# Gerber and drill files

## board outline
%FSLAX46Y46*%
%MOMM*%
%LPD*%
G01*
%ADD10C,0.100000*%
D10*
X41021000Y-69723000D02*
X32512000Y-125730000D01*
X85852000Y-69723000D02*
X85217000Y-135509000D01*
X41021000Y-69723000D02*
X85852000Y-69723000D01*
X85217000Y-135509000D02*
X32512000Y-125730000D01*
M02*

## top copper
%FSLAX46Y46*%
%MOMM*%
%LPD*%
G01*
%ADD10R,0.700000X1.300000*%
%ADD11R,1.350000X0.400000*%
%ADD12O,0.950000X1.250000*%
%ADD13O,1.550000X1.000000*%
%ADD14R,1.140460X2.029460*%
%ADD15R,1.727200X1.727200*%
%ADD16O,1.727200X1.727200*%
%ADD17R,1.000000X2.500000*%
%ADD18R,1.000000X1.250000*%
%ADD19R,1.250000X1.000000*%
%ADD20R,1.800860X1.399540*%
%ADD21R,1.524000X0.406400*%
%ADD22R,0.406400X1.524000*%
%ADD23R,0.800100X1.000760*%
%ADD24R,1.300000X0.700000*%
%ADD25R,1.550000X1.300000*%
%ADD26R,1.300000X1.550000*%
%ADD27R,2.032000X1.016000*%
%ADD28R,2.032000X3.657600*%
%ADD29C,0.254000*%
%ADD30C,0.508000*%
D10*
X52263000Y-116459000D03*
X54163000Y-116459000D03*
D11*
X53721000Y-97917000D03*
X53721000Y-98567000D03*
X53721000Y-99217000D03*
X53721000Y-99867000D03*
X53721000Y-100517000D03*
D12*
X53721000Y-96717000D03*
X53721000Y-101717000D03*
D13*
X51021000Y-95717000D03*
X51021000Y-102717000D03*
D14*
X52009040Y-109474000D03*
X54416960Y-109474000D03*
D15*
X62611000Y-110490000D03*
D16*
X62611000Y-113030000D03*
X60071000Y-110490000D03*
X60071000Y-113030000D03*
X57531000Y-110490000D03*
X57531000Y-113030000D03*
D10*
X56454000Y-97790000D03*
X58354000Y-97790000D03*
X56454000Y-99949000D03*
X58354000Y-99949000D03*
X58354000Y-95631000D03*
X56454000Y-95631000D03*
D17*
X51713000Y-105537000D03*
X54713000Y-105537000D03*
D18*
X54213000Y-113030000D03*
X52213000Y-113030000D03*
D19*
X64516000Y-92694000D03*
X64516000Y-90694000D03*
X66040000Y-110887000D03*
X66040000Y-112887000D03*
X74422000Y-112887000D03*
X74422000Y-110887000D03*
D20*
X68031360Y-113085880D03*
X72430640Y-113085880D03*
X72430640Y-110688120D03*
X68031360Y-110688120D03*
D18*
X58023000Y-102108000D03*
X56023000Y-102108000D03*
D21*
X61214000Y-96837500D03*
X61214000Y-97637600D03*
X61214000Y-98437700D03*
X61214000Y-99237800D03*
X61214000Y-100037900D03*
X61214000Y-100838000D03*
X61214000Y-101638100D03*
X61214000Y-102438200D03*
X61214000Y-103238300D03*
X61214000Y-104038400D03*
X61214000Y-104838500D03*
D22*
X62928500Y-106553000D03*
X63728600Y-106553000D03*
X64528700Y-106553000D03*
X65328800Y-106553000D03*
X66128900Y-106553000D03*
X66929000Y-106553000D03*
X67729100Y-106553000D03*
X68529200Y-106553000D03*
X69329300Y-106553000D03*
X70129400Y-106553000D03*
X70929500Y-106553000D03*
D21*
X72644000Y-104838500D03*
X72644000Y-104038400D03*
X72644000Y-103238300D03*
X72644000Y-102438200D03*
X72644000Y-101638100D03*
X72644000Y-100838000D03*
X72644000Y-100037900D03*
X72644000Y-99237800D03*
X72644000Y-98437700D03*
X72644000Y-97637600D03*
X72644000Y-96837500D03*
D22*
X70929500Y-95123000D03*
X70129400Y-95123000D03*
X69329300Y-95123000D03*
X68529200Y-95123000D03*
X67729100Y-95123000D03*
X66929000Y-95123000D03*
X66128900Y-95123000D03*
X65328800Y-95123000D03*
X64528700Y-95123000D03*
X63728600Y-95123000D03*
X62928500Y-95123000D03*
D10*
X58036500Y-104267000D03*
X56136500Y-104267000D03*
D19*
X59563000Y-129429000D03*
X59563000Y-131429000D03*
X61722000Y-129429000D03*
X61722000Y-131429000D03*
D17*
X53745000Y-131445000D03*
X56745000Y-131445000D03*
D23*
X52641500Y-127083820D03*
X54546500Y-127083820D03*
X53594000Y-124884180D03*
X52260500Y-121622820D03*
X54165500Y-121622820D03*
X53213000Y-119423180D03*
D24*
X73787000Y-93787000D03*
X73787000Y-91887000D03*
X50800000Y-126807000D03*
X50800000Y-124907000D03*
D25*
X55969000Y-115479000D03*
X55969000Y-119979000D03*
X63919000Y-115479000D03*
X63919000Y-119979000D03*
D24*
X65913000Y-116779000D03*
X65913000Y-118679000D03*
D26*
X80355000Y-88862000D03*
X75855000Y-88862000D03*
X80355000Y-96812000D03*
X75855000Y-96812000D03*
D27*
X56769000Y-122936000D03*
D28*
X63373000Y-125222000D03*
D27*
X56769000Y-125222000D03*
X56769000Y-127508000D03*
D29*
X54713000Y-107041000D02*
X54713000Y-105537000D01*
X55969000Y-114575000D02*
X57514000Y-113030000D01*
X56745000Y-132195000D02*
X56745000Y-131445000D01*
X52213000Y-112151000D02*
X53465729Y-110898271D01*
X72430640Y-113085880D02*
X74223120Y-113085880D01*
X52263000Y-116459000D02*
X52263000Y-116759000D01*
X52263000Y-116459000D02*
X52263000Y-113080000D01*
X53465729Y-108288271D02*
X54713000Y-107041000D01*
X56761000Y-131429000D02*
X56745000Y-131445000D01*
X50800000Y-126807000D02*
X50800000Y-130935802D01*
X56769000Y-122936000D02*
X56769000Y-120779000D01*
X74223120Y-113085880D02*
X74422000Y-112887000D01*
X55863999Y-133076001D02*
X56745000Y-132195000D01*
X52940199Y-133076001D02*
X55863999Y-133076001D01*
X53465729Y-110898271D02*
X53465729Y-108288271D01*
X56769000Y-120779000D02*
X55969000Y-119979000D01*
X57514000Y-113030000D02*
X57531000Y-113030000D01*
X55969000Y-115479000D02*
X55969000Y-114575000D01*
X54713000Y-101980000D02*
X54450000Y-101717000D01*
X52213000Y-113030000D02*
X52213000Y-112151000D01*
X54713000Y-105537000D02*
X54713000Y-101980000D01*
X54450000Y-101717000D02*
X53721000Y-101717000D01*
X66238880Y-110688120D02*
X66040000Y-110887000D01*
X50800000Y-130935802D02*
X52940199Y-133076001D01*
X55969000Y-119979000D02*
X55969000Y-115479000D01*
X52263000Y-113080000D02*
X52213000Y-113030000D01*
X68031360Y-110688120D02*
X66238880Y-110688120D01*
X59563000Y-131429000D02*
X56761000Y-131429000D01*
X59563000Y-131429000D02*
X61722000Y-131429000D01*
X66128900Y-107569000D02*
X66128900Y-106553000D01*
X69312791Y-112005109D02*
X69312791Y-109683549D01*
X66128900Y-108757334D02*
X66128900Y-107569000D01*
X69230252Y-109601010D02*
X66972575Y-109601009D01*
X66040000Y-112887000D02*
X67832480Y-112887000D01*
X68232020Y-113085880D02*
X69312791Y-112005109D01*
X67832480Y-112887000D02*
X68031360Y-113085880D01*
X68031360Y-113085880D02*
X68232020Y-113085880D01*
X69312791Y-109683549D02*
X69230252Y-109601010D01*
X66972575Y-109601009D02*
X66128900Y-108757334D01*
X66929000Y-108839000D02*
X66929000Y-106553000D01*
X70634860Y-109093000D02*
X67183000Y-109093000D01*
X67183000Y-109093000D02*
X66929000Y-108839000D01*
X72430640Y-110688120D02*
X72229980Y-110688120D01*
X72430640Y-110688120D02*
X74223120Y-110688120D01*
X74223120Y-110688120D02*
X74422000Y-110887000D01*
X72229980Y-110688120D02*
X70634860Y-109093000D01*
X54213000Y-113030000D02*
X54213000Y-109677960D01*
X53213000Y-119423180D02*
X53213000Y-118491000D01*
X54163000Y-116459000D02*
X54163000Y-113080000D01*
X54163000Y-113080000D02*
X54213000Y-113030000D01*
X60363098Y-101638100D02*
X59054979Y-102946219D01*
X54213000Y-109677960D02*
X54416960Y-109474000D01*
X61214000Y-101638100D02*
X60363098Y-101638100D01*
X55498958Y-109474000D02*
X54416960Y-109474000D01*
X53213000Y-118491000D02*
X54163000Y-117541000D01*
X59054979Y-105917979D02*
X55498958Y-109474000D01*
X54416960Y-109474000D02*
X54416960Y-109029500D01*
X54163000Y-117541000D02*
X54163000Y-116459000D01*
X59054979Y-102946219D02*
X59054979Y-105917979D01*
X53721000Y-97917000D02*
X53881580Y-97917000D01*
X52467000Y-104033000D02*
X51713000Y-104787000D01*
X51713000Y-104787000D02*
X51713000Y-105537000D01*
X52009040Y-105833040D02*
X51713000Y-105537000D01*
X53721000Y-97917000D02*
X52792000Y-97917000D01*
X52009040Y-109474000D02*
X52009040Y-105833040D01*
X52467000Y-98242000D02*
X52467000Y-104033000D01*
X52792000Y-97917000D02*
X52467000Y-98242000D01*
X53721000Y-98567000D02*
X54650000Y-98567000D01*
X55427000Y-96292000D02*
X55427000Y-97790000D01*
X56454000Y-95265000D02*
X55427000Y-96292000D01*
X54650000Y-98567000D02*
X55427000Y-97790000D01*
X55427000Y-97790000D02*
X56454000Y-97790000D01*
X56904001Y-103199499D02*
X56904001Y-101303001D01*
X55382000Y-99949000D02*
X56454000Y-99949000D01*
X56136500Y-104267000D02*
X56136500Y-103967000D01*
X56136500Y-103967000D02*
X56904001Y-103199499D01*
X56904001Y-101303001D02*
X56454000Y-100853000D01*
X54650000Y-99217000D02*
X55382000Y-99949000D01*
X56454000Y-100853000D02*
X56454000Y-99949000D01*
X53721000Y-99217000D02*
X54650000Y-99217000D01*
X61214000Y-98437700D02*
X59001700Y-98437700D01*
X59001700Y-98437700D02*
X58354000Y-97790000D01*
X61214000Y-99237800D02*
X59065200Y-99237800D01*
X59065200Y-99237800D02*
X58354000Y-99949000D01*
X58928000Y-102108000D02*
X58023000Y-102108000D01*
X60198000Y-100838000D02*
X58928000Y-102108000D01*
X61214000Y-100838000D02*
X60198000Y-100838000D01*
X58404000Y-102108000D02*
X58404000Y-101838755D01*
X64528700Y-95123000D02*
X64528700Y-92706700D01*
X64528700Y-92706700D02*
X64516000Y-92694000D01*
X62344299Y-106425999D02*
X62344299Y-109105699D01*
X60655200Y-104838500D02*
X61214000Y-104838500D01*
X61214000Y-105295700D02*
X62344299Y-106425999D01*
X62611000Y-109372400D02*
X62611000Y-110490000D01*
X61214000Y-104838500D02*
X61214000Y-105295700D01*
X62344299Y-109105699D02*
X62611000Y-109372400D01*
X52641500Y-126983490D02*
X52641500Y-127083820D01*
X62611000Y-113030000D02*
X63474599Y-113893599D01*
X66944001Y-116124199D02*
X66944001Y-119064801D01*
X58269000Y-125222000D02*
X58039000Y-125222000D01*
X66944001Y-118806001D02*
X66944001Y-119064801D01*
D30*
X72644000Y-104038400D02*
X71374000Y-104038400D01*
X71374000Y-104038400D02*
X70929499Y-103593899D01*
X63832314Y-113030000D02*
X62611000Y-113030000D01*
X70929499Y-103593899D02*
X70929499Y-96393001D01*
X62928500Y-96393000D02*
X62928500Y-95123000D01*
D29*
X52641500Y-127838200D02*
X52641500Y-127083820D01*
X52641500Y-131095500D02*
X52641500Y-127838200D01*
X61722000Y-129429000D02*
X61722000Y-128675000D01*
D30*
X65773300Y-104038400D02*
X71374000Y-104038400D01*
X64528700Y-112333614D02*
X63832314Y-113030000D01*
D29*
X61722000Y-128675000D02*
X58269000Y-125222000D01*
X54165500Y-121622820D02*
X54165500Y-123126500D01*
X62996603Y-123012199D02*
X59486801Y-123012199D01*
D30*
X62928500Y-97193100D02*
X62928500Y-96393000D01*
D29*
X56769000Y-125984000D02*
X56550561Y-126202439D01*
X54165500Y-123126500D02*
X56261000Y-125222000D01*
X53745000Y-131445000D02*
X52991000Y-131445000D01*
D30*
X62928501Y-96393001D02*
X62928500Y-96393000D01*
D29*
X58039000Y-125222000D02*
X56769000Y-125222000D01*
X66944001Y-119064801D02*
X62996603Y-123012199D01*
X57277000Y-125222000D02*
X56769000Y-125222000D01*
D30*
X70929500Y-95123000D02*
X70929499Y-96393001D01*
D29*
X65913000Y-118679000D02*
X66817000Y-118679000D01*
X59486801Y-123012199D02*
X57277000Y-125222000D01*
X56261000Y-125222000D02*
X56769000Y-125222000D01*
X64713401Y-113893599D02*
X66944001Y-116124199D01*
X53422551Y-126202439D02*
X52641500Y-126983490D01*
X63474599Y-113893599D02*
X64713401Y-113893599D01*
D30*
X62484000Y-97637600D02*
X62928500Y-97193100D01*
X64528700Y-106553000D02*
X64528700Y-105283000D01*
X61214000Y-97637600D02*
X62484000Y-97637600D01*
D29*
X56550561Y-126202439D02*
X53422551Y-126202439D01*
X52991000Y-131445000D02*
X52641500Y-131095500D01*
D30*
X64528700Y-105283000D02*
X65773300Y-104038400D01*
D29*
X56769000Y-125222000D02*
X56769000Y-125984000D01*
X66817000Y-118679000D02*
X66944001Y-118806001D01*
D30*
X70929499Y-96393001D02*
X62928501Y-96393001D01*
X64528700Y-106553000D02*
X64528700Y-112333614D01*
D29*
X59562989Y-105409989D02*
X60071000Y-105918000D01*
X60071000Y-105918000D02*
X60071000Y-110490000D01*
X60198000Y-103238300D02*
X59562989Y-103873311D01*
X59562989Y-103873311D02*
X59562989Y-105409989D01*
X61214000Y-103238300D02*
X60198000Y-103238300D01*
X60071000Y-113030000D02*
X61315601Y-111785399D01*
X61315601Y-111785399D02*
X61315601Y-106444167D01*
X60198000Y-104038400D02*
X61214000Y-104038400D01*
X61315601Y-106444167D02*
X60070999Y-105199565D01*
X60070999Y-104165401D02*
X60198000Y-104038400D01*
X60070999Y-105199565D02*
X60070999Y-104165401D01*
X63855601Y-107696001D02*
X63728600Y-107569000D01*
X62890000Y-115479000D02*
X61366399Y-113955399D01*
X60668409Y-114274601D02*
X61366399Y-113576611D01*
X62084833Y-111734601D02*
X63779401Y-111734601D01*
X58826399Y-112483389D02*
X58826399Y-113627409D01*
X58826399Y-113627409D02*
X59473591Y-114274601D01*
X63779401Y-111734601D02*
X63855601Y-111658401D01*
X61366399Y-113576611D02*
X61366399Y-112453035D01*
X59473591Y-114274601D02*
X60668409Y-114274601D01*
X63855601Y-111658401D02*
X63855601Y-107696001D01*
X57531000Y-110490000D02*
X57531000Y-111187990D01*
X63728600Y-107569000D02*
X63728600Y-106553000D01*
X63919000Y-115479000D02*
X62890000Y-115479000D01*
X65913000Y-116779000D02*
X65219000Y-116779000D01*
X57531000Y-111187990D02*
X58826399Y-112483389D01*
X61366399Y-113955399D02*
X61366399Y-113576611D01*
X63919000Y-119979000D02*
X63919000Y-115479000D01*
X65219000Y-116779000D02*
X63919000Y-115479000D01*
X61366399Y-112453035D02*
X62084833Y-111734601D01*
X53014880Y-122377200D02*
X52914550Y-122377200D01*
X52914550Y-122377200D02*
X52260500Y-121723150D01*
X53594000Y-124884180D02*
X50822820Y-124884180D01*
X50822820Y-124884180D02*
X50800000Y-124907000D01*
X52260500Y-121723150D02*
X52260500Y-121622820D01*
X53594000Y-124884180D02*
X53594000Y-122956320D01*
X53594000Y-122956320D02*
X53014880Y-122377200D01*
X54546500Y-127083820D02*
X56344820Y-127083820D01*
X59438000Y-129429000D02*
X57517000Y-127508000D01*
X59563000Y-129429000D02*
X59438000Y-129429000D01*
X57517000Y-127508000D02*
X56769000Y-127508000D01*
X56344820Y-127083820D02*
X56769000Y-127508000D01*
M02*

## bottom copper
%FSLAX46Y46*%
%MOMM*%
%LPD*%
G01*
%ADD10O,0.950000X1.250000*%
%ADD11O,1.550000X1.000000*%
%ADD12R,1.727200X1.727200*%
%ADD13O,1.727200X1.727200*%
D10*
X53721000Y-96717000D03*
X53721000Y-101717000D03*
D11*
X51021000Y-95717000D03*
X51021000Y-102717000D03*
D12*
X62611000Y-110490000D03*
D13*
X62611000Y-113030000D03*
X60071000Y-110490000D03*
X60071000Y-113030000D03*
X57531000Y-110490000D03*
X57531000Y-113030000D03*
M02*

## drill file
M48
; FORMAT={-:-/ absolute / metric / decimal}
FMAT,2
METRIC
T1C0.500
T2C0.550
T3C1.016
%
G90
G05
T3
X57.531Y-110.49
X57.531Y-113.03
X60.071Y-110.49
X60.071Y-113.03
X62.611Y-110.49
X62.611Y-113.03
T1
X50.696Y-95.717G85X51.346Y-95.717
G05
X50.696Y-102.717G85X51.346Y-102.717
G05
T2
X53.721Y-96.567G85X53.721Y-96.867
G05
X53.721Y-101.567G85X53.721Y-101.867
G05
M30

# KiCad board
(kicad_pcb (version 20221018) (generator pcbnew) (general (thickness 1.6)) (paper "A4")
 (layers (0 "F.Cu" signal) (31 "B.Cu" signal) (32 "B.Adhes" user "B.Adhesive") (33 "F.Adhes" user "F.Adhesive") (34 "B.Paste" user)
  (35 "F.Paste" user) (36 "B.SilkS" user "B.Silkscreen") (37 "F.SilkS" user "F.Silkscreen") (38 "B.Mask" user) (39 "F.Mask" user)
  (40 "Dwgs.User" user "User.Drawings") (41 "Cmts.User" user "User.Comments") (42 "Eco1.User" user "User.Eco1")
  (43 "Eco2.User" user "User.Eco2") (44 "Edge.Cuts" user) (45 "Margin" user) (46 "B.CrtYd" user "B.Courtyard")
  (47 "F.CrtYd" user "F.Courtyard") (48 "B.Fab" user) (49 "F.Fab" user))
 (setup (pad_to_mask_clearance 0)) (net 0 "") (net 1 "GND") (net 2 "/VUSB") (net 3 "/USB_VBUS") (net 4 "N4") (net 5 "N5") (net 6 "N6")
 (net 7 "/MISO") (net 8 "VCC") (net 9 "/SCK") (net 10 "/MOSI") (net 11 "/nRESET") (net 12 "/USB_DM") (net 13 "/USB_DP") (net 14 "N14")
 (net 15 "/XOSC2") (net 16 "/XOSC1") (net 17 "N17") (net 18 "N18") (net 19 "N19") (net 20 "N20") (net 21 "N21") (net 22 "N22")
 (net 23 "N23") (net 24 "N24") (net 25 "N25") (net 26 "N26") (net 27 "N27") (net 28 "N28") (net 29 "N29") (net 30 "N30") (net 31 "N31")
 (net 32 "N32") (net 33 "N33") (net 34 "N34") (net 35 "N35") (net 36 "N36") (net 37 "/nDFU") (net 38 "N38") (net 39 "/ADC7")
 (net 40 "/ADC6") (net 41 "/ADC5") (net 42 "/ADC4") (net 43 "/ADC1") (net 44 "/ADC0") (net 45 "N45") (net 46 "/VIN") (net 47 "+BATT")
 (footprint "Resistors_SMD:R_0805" (layer "F.Cu") (at 53.213 116.459)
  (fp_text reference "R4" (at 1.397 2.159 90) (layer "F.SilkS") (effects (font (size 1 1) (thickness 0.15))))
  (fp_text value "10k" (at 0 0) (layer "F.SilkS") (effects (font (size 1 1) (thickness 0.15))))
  (pad "1" smd rect (at -0.95 0) (size 0.7 1.3) (layers "F.Cu" "F.Paste" "F.Mask") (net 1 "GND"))
  (pad "2" smd rect (at 0.95 0) (size 0.7 1.3) (layers "F.Cu" "F.Paste" "F.Mask") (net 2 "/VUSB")))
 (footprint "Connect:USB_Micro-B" (layer "F.Cu") (at 53.721 97.917)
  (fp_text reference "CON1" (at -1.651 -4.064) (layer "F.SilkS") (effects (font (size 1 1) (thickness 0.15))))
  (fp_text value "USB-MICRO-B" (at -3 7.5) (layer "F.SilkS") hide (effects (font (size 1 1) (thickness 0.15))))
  (pad "1" smd rect (at 0 0) (size 1.35 0.4) (layers "F.Cu" "F.Paste" "F.Mask") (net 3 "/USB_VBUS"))
  (pad "2" smd rect (at 0 0.65) (size 1.35 0.4) (layers "F.Cu" "F.Paste" "F.Mask") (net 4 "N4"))
  (pad "3" smd rect (at 0 1.3) (size 1.35 0.4) (layers "F.Cu" "F.Paste" "F.Mask") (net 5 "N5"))
  (pad "4" smd rect (at 0 1.95) (size 1.35 0.4) (layers "F.Cu" "F.Paste" "F.Mask") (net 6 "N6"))
  (pad "5" smd rect (at 0 2.6) (size 1.35 0.4) (layers "F.Cu" "F.Paste" "F.Mask") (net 1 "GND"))
  (pad "6" thru_hole oval (at 0 -1.2) (size 0.95 1.25) (drill oval 0.55 0.85) (layers "*.Cu" "*.Mask" "F.SilkS") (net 1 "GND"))
  (pad "7" thru_hole oval (at 0 3.8) (size 0.95 1.25) (drill oval 0.55 0.85) (layers "*.Cu" "*.Mask" "F.SilkS") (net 1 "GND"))
  (pad "8" thru_hole oval (at -2.7 -2.2) (size 1.55 1) (drill oval 1.15 0.5) (layers "*.Cu" "*.Mask" "F.SilkS") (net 1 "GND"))
  (pad "9" thru_hole oval (at -2.7 4.8) (size 1.55 1) (drill oval 1.15 0.5) (layers "*.Cu" "*.Mask" "F.SilkS") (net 1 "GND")))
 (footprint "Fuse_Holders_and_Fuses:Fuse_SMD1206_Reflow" (layer "F.Cu") (at 53.213 109.474)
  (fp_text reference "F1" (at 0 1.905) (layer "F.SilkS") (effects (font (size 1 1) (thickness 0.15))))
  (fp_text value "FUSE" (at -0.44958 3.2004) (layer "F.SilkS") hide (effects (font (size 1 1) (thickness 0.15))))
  (pad "1" smd rect (at -1.20396 0 90) (size 2.02946 1.14046) (layers "F.Cu" "F.Paste" "F.Mask") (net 3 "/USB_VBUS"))
  (pad "2" smd rect (at 1.20396 0 90) (size 2.02946 1.14046) (layers "F.Cu" "F.Paste" "F.Mask") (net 2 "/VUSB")))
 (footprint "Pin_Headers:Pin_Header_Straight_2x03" (layer "F.Cu") (at 60.071 111.76 180)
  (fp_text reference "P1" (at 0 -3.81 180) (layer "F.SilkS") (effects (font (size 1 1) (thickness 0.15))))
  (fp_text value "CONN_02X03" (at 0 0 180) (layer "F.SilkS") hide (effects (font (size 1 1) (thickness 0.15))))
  (pad "1" thru_hole rect (at -2.54 1.27 180) (size 1.7272 1.7272) (drill 1.016) (layers "*.Cu" "*.Mask" "F.SilkS") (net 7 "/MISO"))
  (pad "2" thru_hole oval (at -2.54 -1.27 180) (size 1.7272 1.7272) (drill 1.016) (layers "*.Cu" "*.Mask" "F.SilkS") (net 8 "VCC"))
  (pad "3" thru_hole oval (at 0 1.27 180) (size 1.7272 1.7272) (drill 1.016) (layers "*.Cu" "*.Mask" "F.SilkS") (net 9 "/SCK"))
  (pad "4" thru_hole oval (at 0 -1.27 180) (size 1.7272 1.7272) (drill 1.016) (layers "*.Cu" "*.Mask" "F.SilkS") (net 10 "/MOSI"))
  (pad "5" thru_hole oval (at 2.54 1.27 180) (size 1.7272 1.7272) (drill 1.016) (layers "*.Cu" "*.Mask" "F.SilkS") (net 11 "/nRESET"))
  (pad "6" thru_hole oval (at 2.54 -1.27 180) (size 1.7272 1.7272) (drill 1.016) (layers "*.Cu" "*.Mask" "F.SilkS") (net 1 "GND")))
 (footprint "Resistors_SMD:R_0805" (layer "F.Cu") (at 57.404 97.79)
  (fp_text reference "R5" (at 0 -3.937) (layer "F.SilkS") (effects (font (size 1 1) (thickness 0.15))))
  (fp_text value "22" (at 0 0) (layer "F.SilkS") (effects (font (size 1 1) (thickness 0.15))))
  (pad "1" smd rect (at -0.95 0) (size 0.7 1.3) (layers "F.Cu" "F.Paste" "F.Mask") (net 4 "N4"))
  (pad "2" smd rect (at 0.95 0) (size 0.7 1.3) (layers "F.Cu" "F.Paste" "F.Mask") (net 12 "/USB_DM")))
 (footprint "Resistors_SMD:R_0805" (layer "F.Cu") (at 57.404 99.949)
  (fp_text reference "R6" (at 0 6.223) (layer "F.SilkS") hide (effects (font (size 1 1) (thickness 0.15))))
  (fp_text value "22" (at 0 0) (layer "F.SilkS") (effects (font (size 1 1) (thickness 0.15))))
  (pad "1" smd rect (at -0.95 0) (size 0.7 1.3) (layers "F.Cu" "F.Paste" "F.Mask") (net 5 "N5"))
  (pad "2" smd rect (at 0.95 0) (size 0.7 1.3) (layers "F.Cu" "F.Paste" "F.Mask") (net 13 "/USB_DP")))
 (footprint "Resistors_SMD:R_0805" (layer "F.Cu") (at 57.404 95.631 180)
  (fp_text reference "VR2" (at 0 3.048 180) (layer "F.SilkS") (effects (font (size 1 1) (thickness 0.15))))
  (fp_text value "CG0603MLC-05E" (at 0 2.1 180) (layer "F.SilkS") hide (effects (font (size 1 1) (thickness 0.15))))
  (pad "1" smd rect (at -0.95 0 180) (size 0.7 1.3) (layers "F.Cu" "F.Paste" "F.Mask") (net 1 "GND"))
  (pad "2" smd rect (at 0.95 0 180) (size 0.7 1.3) (layers "F.Cu" "F.Paste" "F.Mask") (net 4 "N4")))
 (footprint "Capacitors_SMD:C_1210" (layer "F.Cu") (at 53.213 105.537)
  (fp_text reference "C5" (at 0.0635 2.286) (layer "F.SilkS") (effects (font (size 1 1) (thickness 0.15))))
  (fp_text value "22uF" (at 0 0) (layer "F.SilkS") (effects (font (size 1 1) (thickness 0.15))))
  (pad "1" smd rect (at -1.5 0) (size 1 2.5) (layers "F.Cu" "F.Paste" "F.Mask") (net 3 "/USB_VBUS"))
  (pad "2" smd rect (at 1.5 0) (size 1 2.5) (layers "F.Cu" "F.Paste" "F.Mask") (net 1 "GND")))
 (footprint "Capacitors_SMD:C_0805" (layer "F.Cu") (at 53.213 113.03 180)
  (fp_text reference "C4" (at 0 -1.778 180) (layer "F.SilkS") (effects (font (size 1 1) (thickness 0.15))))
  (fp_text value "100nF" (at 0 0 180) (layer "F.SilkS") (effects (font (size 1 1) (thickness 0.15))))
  (pad "1" smd rect (at -1 0 180) (size 1 1.25) (layers "F.Cu" "F.Paste" "F.Mask") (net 2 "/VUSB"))
  (pad "2" smd rect (at 1 0 180) (size 1 1.25) (layers "F.Cu" "F.Paste" "F.Mask") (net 1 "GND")))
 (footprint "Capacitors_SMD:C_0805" (layer "F.Cu") (at 64.516 91.694 90)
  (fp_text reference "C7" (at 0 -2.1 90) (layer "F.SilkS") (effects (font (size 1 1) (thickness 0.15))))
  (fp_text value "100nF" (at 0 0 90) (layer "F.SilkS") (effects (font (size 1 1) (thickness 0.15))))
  (pad "1" smd rect (at -1 0 90) (size 1 1.25) (layers "F.Cu" "F.Paste" "F.Mask") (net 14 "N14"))
  (pad "2" smd rect (at 1 0 90) (size 1 1.25) (layers "F.Cu" "F.Paste" "F.Mask") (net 1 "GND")))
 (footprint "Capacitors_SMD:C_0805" (layer "F.Cu") (at 66.04 111.887 -90)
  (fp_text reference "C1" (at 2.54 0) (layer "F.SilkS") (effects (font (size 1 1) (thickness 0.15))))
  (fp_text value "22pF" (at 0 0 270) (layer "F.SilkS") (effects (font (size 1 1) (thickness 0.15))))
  (pad "1" smd rect (at -1 0 270) (size 1 1.25) (layers "F.Cu" "F.Paste" "F.Mask") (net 1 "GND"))
  (pad "2" smd rect (at 1 0 270) (size 1 1.25) (layers "F.Cu" "F.Paste" "F.Mask") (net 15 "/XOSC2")))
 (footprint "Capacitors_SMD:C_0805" (layer "F.Cu") (at 74.422 111.887 90)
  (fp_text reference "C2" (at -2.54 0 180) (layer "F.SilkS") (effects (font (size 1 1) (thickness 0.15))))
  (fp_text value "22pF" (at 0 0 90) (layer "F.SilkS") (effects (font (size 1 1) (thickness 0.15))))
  (pad "1" smd rect (at -1 0 90) (size 1 1.25) (layers "F.Cu" "F.Paste" "F.Mask") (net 1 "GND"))
  (pad "2" smd rect (at 1 0 90) (size 1 1.25) (layers "F.Cu" "F.Paste" "F.Mask") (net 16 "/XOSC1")))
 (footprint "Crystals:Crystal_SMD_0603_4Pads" (layer "F.Cu") (at 70.231 111.887)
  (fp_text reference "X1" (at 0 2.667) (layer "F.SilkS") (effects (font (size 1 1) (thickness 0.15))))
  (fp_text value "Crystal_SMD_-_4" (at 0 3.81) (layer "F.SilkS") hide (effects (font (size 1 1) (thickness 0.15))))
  (pad "1" smd rect (at -2.19964 1.19888) (size 1.80086 1.39954) (layers "F.Cu" "F.Paste" "F.Mask") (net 15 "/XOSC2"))
  (pad "2" smd rect (at 2.19964 1.19888) (size 1.80086 1.39954) (layers "F.Cu" "F.Paste" "F.Mask") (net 1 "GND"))
  (pad "3" smd rect (at 2.19964 -1.19888) (size 1.80086 1.39954) (layers "F.Cu" "F.Paste" "F.Mask") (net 16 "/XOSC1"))
  (pad "4" smd rect (at -2.19964 -1.19888) (size 1.80086 1.39954) (layers "F.Cu" "F.Paste" "F.Mask") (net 1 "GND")))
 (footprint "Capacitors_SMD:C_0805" (layer "F.Cu") (at 57.023 102.108 180)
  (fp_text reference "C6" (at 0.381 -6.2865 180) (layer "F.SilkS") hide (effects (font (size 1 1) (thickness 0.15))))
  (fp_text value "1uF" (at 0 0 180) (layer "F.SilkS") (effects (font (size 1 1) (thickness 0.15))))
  (pad "1" smd rect (at -1 0 180) (size 1 1.25) (layers "F.Cu" "F.Paste" "F.Mask") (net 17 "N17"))
  (pad "2" smd rect (at 1 0 180) (size 1 1.25) (layers "F.Cu" "F.Paste" "F.Mask") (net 1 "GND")))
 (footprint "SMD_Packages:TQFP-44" (layer "F.Cu") (at 66.929 100.838)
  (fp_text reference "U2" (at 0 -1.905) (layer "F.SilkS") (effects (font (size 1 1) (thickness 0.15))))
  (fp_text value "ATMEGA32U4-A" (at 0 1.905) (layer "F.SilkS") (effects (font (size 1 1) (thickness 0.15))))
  (pad "1" smd rect (at -5.715 -4.0005) (size 1.524 0.4064) (layers "F.Cu" "F.Paste" "F.Mask") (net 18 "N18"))
  (pad "2" smd rect (at -5.715 -3.2004) (size 1.524 0.4064) (layers "F.Cu" "F.Paste" "F.Mask") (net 8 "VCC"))
  (pad "3" smd rect (at -5.715 -2.4003) (size 1.524 0.4064) (layers "F.Cu" "F.Paste" "F.Mask") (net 12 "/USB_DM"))
  (pad "4" smd rect (at -5.715 -1.6002) (size 1.524 0.4064) (layers "F.Cu" "F.Paste" "F.Mask") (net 13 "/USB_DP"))
  (pad "5" smd rect (at -5.715 -0.8001) (size 1.524 0.4064) (layers "F.Cu" "F.Paste" "F.Mask") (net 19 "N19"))
  (pad "6" smd rect (at -5.715 0) (size 1.524 0.4064) (layers "F.Cu" "F.Paste" "F.Mask") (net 17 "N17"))
  (pad "7" smd rect (at -5.715 0.8001) (size 1.524 0.4064) (layers "F.Cu" "F.Paste" "F.Mask") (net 2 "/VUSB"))
  (pad "8" smd rect (at -5.715 1.6002) (size 1.524 0.4064) (layers "F.Cu" "F.Paste" "F.Mask") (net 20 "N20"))
  (pad "9" smd rect (at -5.715 2.4003) (size 1.524 0.4064) (layers "F.Cu" "F.Paste" "F.Mask") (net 9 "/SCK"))
  (pad "10" smd rect (at -5.715 3.2004) (size 1.524 0.4064) (layers "F.Cu" "F.Paste" "F.Mask") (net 10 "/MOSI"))
  (pad "11" smd rect (at -5.715 4.0005) (size 1.524 0.4064) (layers "F.Cu" "F.Paste" "F.Mask") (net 7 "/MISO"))
  (pad "12" smd rect (at -4.0005 5.715) (size 0.4064 1.524) (layers "F.Cu" "F.Paste" "F.Mask") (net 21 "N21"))
  (pad "13" smd rect (at -3.2004 5.715) (size 0.4064 1.524) (layers "F.Cu" "F.Paste" "F.Mask") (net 11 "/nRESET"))
  (pad "14" smd rect (at -2.4003 5.715) (size 0.4064 1.524) (layers "F.Cu" "F.Paste" "F.Mask") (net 8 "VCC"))
  (pad "15" smd rect (at -1.6002 5.715) (size 0.4064 1.524) (layers "F.Cu" "F.Paste" "F.Mask") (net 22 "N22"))
  (pad "16" smd rect (at -0.8001 5.715) (size 0.4064 1.524) (layers "F.Cu" "F.Paste" "F.Mask") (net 15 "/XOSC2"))
  (pad "17" smd rect (at 0 5.715) (size 0.4064 1.524) (layers "F.Cu" "F.Paste" "F.Mask") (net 16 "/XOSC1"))
  (pad "18" smd rect (at 0.8001 5.715) (size 0.4064 1.524) (layers "F.Cu" "F.Paste" "F.Mask") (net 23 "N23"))
  (pad "19" smd rect (at 1.6002 5.715) (size 0.4064 1.524) (layers "F.Cu" "F.Paste" "F.Mask") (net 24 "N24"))
  (pad "20" smd rect (at 2.4003 5.715) (size 0.4064 1.524) (layers "F.Cu" "F.Paste" "F.Mask") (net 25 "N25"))
  (pad "21" smd rect (at 3.2004 5.715) (size 0.4064 1.524) (layers "F.Cu" "F.Paste" "F.Mask") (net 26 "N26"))
  (pad "22" smd rect (at 4.0005 5.715) (size 0.4064 1.524) (layers "F.Cu" "F.Paste" "F.Mask") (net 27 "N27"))
  (pad "23" smd rect (at 5.715 4.0005) (size 1.524 0.4064) (layers "F.Cu" "F.Paste" "F.Mask") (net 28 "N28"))
  (pad "24" smd rect (at 5.715 3.2004) (size 1.524 0.4064) (layers "F.Cu" "F.Paste" "F.Mask") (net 8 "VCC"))
  (pad "25" smd rect (at 5.715 2.4003) (size 1.524 0.4064) (layers "F.Cu" "F.Paste" "F.Mask") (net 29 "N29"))
  (pad "26" smd rect (at 5.715 1.6002) (size 1.524 0.4064) (layers "F.Cu" "F.Paste" "F.Mask") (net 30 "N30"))
  (pad "27" smd rect (at 5.715 0.8001) (size 1.524 0.4064) (layers "F.Cu" "F.Paste" "F.Mask") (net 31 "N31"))
  (pad "28" smd rect (at 5.715 0) (size 1.524 0.4064) (layers "F.Cu" "F.Paste" "F.Mask") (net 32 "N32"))
  (pad "29" smd rect (at 5.715 -0.8001) (size 1.524 0.4064) (layers "F.Cu" "F.Paste" "F.Mask") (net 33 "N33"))
  (pad "30" smd rect (at 5.715 -1.6002) (size 1.524 0.4064) (layers "F.Cu" "F.Paste" "F.Mask") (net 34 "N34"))
  (pad "31" smd rect (at 5.715 -2.4003) (size 1.524 0.4064) (layers "F.Cu" "F.Paste" "F.Mask") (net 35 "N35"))
  (pad "32" smd rect (at 5.715 -3.2004) (size 1.524 0.4064) (layers "F.Cu" "F.Paste" "F.Mask") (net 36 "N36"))
  (pad "33" smd rect (at 5.715 -4.0005) (size 1.524 0.4064) (layers "F.Cu" "F.Paste" "F.Mask") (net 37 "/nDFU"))
  (pad "34" smd rect (at 4.0005 -5.715) (size 0.4064 1.524) (layers "F.Cu" "F.Paste" "F.Mask") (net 8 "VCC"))
  (pad "35" smd rect (at 3.2004 -5.715) (size 0.4064 1.524) (layers "F.Cu" "F.Paste" "F.Mask") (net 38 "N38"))
  (pad "36" smd rect (at 2.4003 -5.715) (size 0.4064 1.524) (layers "F.Cu" "F.Paste" "F.Mask") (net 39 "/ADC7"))
  (pad "37" smd rect (at 1.6002 -5.715) (size 0.4064 1.524) (layers "F.Cu" "F.Paste" "F.Mask") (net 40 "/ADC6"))
  (pad "38" smd rect (at 0.8001 -5.715) (size 0.4064 1.524) (layers "F.Cu" "F.Paste" "F.Mask") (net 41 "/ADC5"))
  (pad "39" smd rect (at 0 -5.715) (size 0.4064 1.524) (layers "F.Cu" "F.Paste" "F.Mask") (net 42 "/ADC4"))
  (pad "40" smd rect (at -0.8001 -5.715) (size 0.4064 1.524) (layers "F.Cu" "F.Paste" "F.Mask") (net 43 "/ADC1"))
  (pad "41" smd rect (at -1.6002 -5.715) (size 0.4064 1.524) (layers "F.Cu" "F.Paste" "F.Mask") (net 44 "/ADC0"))
  (pad "42" smd rect (at -2.4003 -5.715) (size 0.4064 1.524) (layers "F.Cu" "F.Paste" "F.Mask") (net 14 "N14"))
  (pad "43" smd rect (at -3.2004 -5.715) (size 0.4064 1.524) (layers "F.Cu" "F.Paste" "F.Mask") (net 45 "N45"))
  (pad "44" smd rect (at -4.0005 -5.715) (size 0.4064 1.524) (layers "F.Cu" "F.Paste" "F.Mask") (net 8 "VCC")))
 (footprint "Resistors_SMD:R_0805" (layer "F.Cu") (at 57.0865 104.267 180)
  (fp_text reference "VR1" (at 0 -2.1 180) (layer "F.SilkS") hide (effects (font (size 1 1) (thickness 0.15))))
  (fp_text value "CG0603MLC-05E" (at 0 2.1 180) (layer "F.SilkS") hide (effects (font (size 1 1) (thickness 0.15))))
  (pad "1" smd rect (at -0.95 0 180) (size 0.7 1.3) (layers "F.Cu" "F.Paste" "F.Mask") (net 1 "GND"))
  (pad "2" smd rect (at 0.95 0 180) (size 0.7 1.3) (layers "F.Cu" "F.Paste" "F.Mask") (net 5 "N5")))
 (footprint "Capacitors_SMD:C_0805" (layer "F.Cu") (at 59.563 130.429 -90)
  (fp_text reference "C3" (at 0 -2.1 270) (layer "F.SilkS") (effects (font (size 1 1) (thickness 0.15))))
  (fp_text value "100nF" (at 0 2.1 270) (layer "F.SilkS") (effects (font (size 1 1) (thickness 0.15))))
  (pad "1" smd rect (at -1 0 270) (size 1 1.25) (layers "F.Cu" "F.Paste" "F.Mask") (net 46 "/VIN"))
  (pad "2" smd rect (at 1 0 270) (size 1 1.25) (layers "F.Cu" "F.Paste" "F.Mask") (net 1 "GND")))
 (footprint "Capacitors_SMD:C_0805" (layer "F.Cu") (at 61.722 130.429 -90)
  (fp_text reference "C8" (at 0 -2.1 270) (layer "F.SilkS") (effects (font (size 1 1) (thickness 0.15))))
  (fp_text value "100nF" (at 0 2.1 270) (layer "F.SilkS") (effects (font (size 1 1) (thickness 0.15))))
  (pad "1" smd rect (at -1 0 270) (size 1 1.25) (layers "F.Cu" "F.Paste" "F.Mask") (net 8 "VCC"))
  (pad "2" smd rect (at 1 0 270) (size 1 1.25) (layers "F.Cu" "F.Paste" "F.Mask") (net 1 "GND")))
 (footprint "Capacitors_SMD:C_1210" (layer "F.Cu") (at 55.245 131.445)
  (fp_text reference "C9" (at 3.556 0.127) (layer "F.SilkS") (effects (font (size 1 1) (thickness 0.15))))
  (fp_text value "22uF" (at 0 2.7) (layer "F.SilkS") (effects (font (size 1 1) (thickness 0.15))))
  (pad "1" smd rect (at -1.5 0) (size 1 2.5) (layers "F.Cu" "F.Paste" "F.Mask") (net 8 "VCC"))
  (pad "2" smd rect (at 1.5 0) (size 1 2.5) (layers "F.Cu" "F.Paste" "F.Mask") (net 1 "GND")))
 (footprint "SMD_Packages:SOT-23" (layer "F.Cu") (at 53.594 125.984)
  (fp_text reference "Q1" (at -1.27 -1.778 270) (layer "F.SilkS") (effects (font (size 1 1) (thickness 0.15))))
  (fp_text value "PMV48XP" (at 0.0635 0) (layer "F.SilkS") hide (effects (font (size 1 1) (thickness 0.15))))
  (pad "1" smd rect (at -0.9525 1.09982) (size 0.8001 1.00076) (layers "F.Cu" "F.Paste" "F.Mask") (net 8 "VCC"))
  (pad "2" smd rect (at 0.9525 1.09982) (size 0.8001 1.00076) (layers "F.Cu" "F.Paste" "F.Mask") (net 46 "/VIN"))
  (pad "3" smd rect (at 0 -1.09982) (size 0.8001 1.00076) (layers "F.Cu" "F.Paste" "F.Mask") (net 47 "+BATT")))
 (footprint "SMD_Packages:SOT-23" (layer "F.Cu") (at 53.213 120.523)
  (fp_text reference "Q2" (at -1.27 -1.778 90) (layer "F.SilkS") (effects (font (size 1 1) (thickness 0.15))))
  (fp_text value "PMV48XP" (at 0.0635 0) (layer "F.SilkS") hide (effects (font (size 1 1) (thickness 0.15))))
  (pad "1" smd rect (at -0.9525 1.09982) (size 0.8001 1.00076) (layers "F.Cu" "F.Paste" "F.Mask") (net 47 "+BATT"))
  (pad "2" smd rect (at 0.9525 1.09982) (size 0.8001 1.00076) (layers "F.Cu" "F.Paste" "F.Mask") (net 8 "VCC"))
  (pad "3" smd rect (at 0 -1.09982) (size 0.8001 1.00076) (layers "F.Cu" "F.Paste" "F.Mask") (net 2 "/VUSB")))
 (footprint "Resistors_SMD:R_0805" (layer "F.Cu") (at 73.787 92.837 90)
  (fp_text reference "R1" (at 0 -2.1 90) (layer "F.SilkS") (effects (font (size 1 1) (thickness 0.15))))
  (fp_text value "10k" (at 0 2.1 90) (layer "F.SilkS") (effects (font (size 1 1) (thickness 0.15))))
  (pad "1" smd rect (at -0.95 0 90) (size 0.7 1.3) (layers "F.Cu" "F.Paste" "F.Mask") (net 37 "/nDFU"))
  (pad "2" smd rect (at 0.95 0 90) (size 0.7 1.3) (layers "F.Cu" "F.Paste" "F.Mask") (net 8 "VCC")))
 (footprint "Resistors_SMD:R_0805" (layer "F.Cu") (at 50.8 125.857 90)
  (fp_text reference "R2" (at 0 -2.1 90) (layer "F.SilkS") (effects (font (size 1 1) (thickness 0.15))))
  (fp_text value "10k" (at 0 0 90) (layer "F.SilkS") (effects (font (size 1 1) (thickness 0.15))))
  (pad "1" smd rect (at -0.95 0 90) (size 0.7 1.3) (layers "F.Cu" "F.Paste" "F.Mask") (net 1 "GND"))
  (pad "2" smd rect (at 0.95 0 90) (size 0.7 1.3) (layers "F.Cu" "F.Paste" "F.Mask") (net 47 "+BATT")))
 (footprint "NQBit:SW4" (layer "F.Cu") (at 59.944 117.729)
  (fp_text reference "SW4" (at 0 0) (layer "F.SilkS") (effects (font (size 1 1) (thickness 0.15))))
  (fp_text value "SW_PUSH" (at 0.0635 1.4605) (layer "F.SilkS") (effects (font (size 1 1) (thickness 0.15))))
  (pad "1" smd rect (at -3.975 -2.25) (size 1.55 1.3) (layers "F.Cu" "F.Paste" "F.Mask") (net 1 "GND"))
  (pad "1" smd rect (at -3.975 2.25) (size 1.55 1.3) (layers "F.Cu" "F.Paste" "F.Mask") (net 1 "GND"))
  (pad "2" smd rect (at 3.975 -2.25) (size 1.55 1.3) (layers "F.Cu" "F.Paste" "F.Mask") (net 11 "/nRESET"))
  (pad "2" smd rect (at 3.975 2.25) (size 1.55 1.3) (layers "F.Cu" "F.Paste" "F.Mask") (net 11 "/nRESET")))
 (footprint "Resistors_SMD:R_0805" (layer "F.Cu") (at 65.913 117.729 -90)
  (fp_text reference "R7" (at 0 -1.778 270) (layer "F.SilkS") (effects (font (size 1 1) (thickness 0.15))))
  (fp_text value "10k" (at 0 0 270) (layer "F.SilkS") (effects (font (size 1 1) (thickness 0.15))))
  (pad "1" smd rect (at -0.95 0 270) (size 0.7 1.3) (layers "F.Cu" "F.Paste" "F.Mask") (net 11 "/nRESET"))
  (pad "2" smd rect (at 0.95 0 270) (size 0.7 1.3) (layers "F.Cu" "F.Paste" "F.Mask") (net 8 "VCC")))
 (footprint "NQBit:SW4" (layer "F.Cu") (at 78.105 92.837 -90)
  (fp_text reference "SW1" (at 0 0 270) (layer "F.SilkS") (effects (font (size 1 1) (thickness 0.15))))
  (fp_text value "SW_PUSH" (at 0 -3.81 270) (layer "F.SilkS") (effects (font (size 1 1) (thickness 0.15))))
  (pad "1" smd rect (at -3.975 -2.25 270) (size 1.55 1.3) (layers "F.Cu" "F.Paste" "F.Mask") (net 1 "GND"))
  (pad "1" smd rect (at -3.975 2.25 270) (size 1.55 1.3) (layers "F.Cu" "F.Paste" "F.Mask") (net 1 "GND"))
  (pad "2" smd rect (at 3.975 -2.25 270) (size 1.55 1.3) (layers "F.Cu" "F.Paste" "F.Mask") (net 37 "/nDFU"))
  (pad "2" smd rect (at 3.975 2.25 270) (size 1.55 1.3) (layers "F.Cu" "F.Paste" "F.Mask") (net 37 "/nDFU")))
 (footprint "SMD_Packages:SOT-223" (layer "F.Cu") (at 60.071 125.222 -90)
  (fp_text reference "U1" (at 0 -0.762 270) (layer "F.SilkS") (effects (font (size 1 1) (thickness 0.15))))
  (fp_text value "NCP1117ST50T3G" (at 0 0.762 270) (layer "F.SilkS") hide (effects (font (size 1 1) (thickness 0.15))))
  (pad "1" smd rect (at -2.286 3.302 270) (size 1.016 2.032) (layers "F.Cu" "F.Paste" "F.Mask") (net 1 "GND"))
  (pad "2" smd rect (at 0 -3.302 270) (size 3.6576 2.032) (layers "F.Cu" "F.Paste" "F.Mask"))
  (pad "2" smd rect (at 0 3.302 270) (size 1.016 2.032) (layers "F.Cu" "F.Paste" "F.Mask") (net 8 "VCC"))
  (pad "3" smd rect (at 2.286 3.302 270) (size 1.016 2.032) (layers "F.Cu" "F.Paste" "F.Mask") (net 46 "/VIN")))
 (gr_line (start 41.021 69.723) (end 32.512 125.73) (stroke (width 0.1) (type solid)) (layer "Edge.Cuts"))
 (gr_line (start 85.852 69.723) (end 85.217 135.509) (stroke (width 0.1) (type solid)) (layer "Edge.Cuts"))
 (gr_line (start 41.021 69.723) (end 85.852 69.723) (stroke (width 0.1) (type solid)) (layer "Edge.Cuts"))
 (gr_line (start 85.217 135.509) (end 32.512 125.73) (stroke (width 0.1) (type solid)) (layer "Edge.Cuts"))
 (segment (start 54.713 107.041) (end 54.713 105.537) (width 0.254) (layer "F.Cu") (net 1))
 (segment (start 55.969 114.575) (end 57.514 113.03) (width 0.254) (layer "F.Cu") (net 1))
 (segment (start 56.745 132.195) (end 56.745 131.445) (width 0.254) (layer "F.Cu") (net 1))
 (segment (start 52.213 112.151) (end 53.465729 110.898271) (width 0.254) (layer "F.Cu") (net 1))
 (segment (start 72.43064 113.08588) (end 74.22312 113.08588) (width 0.254) (layer "F.Cu") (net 1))
 (segment (start 52.263 116.459) (end 52.263 116.759) (width 0.254) (layer "F.Cu") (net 1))
 (segment (start 52.263 116.459) (end 52.263 113.08) (width 0.254) (layer "F.Cu") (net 1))
 (segment (start 53.465729 108.288271) (end 54.713 107.041) (width 0.254) (layer "F.Cu") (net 1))
 (segment (start 56.761 131.429) (end 56.745 131.445) (width 0.254) (layer "F.Cu") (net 1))
 (segment (start 50.8 126.807) (end 50.8 130.935802) (width 0.254) (layer "F.Cu") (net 1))
 (segment (start 56.769 122.936) (end 56.769 120.779) (width 0.254) (layer "F.Cu") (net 1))
 (segment (start 74.22312 113.08588) (end 74.422 112.887) (width 0.254) (layer "F.Cu") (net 1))
 (segment (start 55.863999 133.076001) (end 56.745 132.195) (width 0.254) (layer "F.Cu") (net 1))
 (segment (start 52.940199 133.076001) (end 55.863999 133.076001) (width 0.254) (layer "F.Cu") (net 1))
 (segment (start 53.465729 110.898271) (end 53.465729 108.288271) (width 0.254) (layer "F.Cu") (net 1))
 (segment (start 56.769 120.779) (end 55.969 119.979) (width 0.254) (layer "F.Cu") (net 1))
 (segment (start 57.514 113.03) (end 57.531 113.03) (width 0.254) (layer "F.Cu") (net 1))
 (segment (start 55.969 115.479) (end 55.969 114.575) (width 0.254) (layer "F.Cu") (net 1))
 (segment (start 54.713 101.98) (end 54.45 101.717) (width 0.254) (layer "F.Cu") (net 1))
 (segment (start 52.213 113.03) (end 52.213 112.151) (width 0.254) (layer "F.Cu") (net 1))
 (segment (start 54.713 105.537) (end 54.713 101.98) (width 0.254) (layer "F.Cu") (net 1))
 (segment (start 54.45 101.717) (end 53.721 101.717) (width 0.254) (layer "F.Cu") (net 1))
 (segment (start 66.23888 110.68812) (end 66.04 110.887) (width 0.254) (layer "F.Cu") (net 1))
 (segment (start 50.8 130.935802) (end 52.940199 133.076001) (width 0.254) (layer "F.Cu") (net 1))
 (segment (start 55.969 119.979) (end 55.969 115.479) (width 0.254) (layer "F.Cu") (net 1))
 (segment (start 52.263 113.08) (end 52.213 113.03) (width 0.254) (layer "F.Cu") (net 1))
 (segment (start 68.03136 110.68812) (end 66.23888 110.68812) (width 0.254) (layer "F.Cu") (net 1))
 (segment (start 59.563 131.429) (end 56.761 131.429) (width 0.254) (layer "F.Cu") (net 1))
 (segment (start 59.563 131.429) (end 61.722 131.429) (width 0.254) (layer "F.Cu") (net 1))
 (segment (start 66.1289 107.569) (end 66.1289 106.553) (width 0.254) (layer "F.Cu") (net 15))
 (segment (start 69.312791 112.005109) (end 69.312791 109.683549) (width 0.254) (layer "F.Cu") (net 15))
 (segment (start 66.1289 108.757334) (end 66.1289 107.569) (width 0.254) (layer "F.Cu") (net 15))
 (segment (start 69.230252 109.60101) (end 66.972575 109.601009) (width 0.254) (layer "F.Cu") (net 15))
 (segment (start 66.04 112.887) (end 67.83248 112.887) (width 0.254) (layer "F.Cu") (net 15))
 (segment (start 68.23202 113.08588) (end 69.312791 112.005109) (width 0.254) (layer "F.Cu") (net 15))
 (segment (start 67.83248 112.887) (end 68.03136 113.08588) (width 0.254) (layer "F.Cu") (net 15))
 (segment (start 68.03136 113.08588) (end 68.23202 113.08588) (width 0.254) (layer "F.Cu") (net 15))
 (segment (start 69.312791 109.683549) (end 69.230252 109.60101) (width 0.254) (layer "F.Cu") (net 15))
 (segment (start 66.972575 109.601009) (end 66.1289 108.757334) (width 0.254) (layer "F.Cu") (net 15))
 (segment (start 66.929 108.839) (end 66.929 106.553) (width 0.254) (layer "F.Cu") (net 16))
 (segment (start 70.63486 109.093) (end 67.183 109.093) (width 0.254) (layer "F.Cu") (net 16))
 (segment (start 67.183 109.093) (end 66.929 108.839) (width 0.254) (layer "F.Cu") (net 16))
 (segment (start 72.43064 110.68812) (end 72.22998 110.68812) (width 0.254) (layer "F.Cu") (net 16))
 (segment (start 72.43064 110.68812) (end 74.22312 110.68812) (width 0.254) (layer "F.Cu") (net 16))
 (segment (start 74.22312 110.68812) (end 74.422 110.887) (width 0.254) (layer "F.Cu") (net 16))
 (segment (start 72.22998 110.68812) (end 70.63486 109.093) (width 0.254) (layer "F.Cu") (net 16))
 (segment (start 54.213 113.03) (end 54.213 109.67796) (width 0.254) (layer "F.Cu") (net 2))
 (segment (start 53.213 119.42318) (end 53.213 118.491) (width 0.254) (layer "F.Cu") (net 2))
 (segment (start 54.163 116.459) (end 54.163 113.08) (width 0.254) (layer "F.Cu") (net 2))
 (segment (start 54.163 113.08) (end 54.213 113.03) (width 0.254) (layer "F.Cu") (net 2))
 (segment (start 60.363098 101.6381) (end 59.054979 102.946219) (width 0.254) (layer "F.Cu") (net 2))
 (segment (start 54.213 109.67796) (end 54.41696 109.474) (width 0.254) (layer "F.Cu") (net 2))
 (segment (start 61.214 101.6381) (end 60.363098 101.6381) (width 0.254) (layer "F.Cu") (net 2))
 (segment (start 55.498958 109.474) (end 54.41696 109.474) (width 0.254) (layer "F.Cu") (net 2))
 (segment (start 53.213 118.491) (end 54.163 117.541) (width 0.254) (layer "F.Cu") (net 2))
 (segment (start 59.054979 105.917979) (end 55.498958 109.474) (width 0.254) (layer "F.Cu") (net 2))
 (segment (start 54.41696 109.474) (end 54.41696 109.0295) (width 0.254) (layer "F.Cu") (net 2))
 (segment (start 54.163 117.541) (end 54.163 116.459) (width 0.254) (layer "F.Cu") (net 2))
 (segment (start 59.054979 102.946219) (end 59.054979 105.917979) (width 0.254) (layer "F.Cu") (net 2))
 (segment (start 53.721 97.917) (end 53.88158 97.917) (width 0.254) (layer "F.Cu") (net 3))
 (segment (start 52.467 104.033) (end 51.713 104.787) (width 0.254) (layer "F.Cu") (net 3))
 (segment (start 51.713 104.787) (end 51.713 105.537) (width 0.254) (layer "F.Cu") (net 3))
 (segment (start 52.00904 105.83304) (end 51.713 105.537) (width 0.254) (layer "F.Cu") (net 3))
 (segment (start 53.721 97.917) (end 52.792 97.917) (width 0.254) (layer "F.Cu") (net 3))
 (segment (start 52.00904 109.474) (end 52.00904 105.83304) (width 0.254) (layer "F.Cu") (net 3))
 (segment (start 52.467 98.242) (end 52.467 104.033) (width 0.254) (layer "F.Cu") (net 3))
 (segment (start 52.792 97.917) (end 52.467 98.242) (width 0.254) (layer "F.Cu") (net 3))
 (segment (start 53.721 98.567) (end 54.65 98.567) (width 0.254) (layer "F.Cu") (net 4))
 (segment (start 55.427 96.292) (end 55.427 97.79) (width 0.254) (layer "F.Cu") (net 4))
 (segment (start 56.454 95.265) (end 55.427 96.292) (width 0.254) (layer "F.Cu") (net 4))
 (segment (start 54.65 98.567) (end 55.427 97.79) (width 0.254) (layer "F.Cu") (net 4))
 (segment (start 55.427 97.79) (end 56.454 97.79) (width 0.254) (layer "F.Cu") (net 4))
 (segment (start 56.904001 103.199499) (end 56.904001 101.303001) (width 0.254) (layer "F.Cu") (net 5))
 (segment (start 55.382 99.949) (end 56.454 99.949) (width 0.254) (layer "F.Cu") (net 5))
 (segment (start 56.1365 104.267) (end 56.1365 103.967) (width 0.254) (layer "F.Cu") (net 5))
 (segment (start 56.1365 103.967) (end 56.904001 103.199499) (width 0.254) (layer "F.Cu") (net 5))
 (segment (start 56.904001 101.303001) (end 56.454 100.853) (width 0.254) (layer "F.Cu") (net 5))
 (segment (start 54.65 99.217) (end 55.382 99.949) (width 0.254) (layer "F.Cu") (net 5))
 (segment (start 56.454 100.853) (end 56.454 99.949) (width 0.254) (layer "F.Cu") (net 5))
 (segment (start 53.721 99.217) (end 54.65 99.217) (width 0.254) (layer "F.Cu") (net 5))
 (segment (start 61.214 98.4377) (end 59.0017 98.4377) (width 0.254) (layer "F.Cu") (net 12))
 (segment (start 59.0017 98.4377) (end 58.354 97.79) (width 0.254) (layer "F.Cu") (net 12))
 (segment (start 61.214 99.2378) (end 59.0652 99.2378) (width 0.254) (layer "F.Cu") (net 13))
 (segment (start 59.0652 99.2378) (end 58.354 99.949) (width 0.254) (layer "F.Cu") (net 13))
 (segment (start 58.928 102.108) (end 58.023 102.108) (width 0.254) (layer "F.Cu") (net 17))
 (segment (start 60.198 100.838) (end 58.928 102.108) (width 0.254) (layer "F.Cu") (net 17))
 (segment (start 61.214 100.838) (end 60.198 100.838) (width 0.254) (layer "F.Cu") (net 17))
 (segment (start 58.404 102.108) (end 58.404 101.838755) (width 0.254) (layer "F.Cu") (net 17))
 (segment (start 64.5287 95.123) (end 64.5287 92.7067) (width 0.254) (layer "F.Cu") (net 14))
 (segment (start 64.5287 92.7067) (end 64.516 92.694) (width 0.254) (layer "F.Cu") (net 14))
 (segment (start 62.344299 106.425999) (end 62.344299 109.105699) (width 0.254) (layer "F.Cu") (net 7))
 (segment (start 60.6552 104.8385) (end 61.214 104.8385) (width 0.254) (layer "F.Cu") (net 7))
 (segment (start 61.214 105.2957) (end 62.344299 106.425999) (width 0.254) (layer "F.Cu") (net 7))
 (segment (start 62.611 109.3724) (end 62.611 110.49) (width 0.254) (layer "F.Cu") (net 7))
 (segment (start 61.214 104.8385) (end 61.214 105.2957) (width 0.254) (layer "F.Cu") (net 7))
 (segment (start 62.344299 109.105699) (end 62.611 109.3724) (width 0.254) (layer "F.Cu") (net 7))
 (segment (start 52.6415 126.98349) (end 52.6415 127.08382) (width 0.254) (layer "F.Cu") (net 8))
 (segment (start 62.611 113.03) (end 63.474599 113.893599) (width 0.254) (layer "F.Cu") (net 8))
 (segment (start 66.944001 116.124199) (end 66.944001 119.064801) (width 0.254) (layer "F.Cu") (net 8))
 (segment (start 58.269 125.222) (end 58.039 125.222) (width 0.254) (layer "F.Cu") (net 8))
 (segment (start 66.944001 118.806001) (end 66.944001 119.064801) (width 0.254) (layer "F.Cu") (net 8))
 (segment (start 72.644 104.0384) (end 71.374 104.0384) (width 0.508) (layer "F.Cu") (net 8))
 (segment (start 71.374 104.0384) (end 70.929499 103.593899) (width 0.508) (layer "F.Cu") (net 8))
 (segment (start 63.832314 113.03) (end 62.611 113.03) (width 0.508) (layer "F.Cu") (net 8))
 (segment (start 70.929499 103.593899) (end 70.929499 96.393001) (width 0.508) (layer "F.Cu") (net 8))
 (segment (start 62.9285 96.393) (end 62.9285 95.123) (width 0.508) (layer "F.Cu") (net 8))
 (segment (start 52.6415 127.8382) (end 52.6415 127.08382) (width 0.254) (layer "F.Cu") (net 8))
 (segment (start 52.6415 131.0955) (end 52.6415 127.8382) (width 0.254) (layer "F.Cu") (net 8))
 (segment (start 61.722 129.429) (end 61.722 128.675) (width 0.254) (layer "F.Cu") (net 8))
 (segment (start 65.7733 104.0384) (end 71.374 104.0384) (width 0.508) (layer "F.Cu") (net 8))
 (segment (start 64.5287 112.333614) (end 63.832314 113.03) (width 0.508) (layer "F.Cu") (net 8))
 (segment (start 61.722 128.675) (end 58.269 125.222) (width 0.254) (layer "F.Cu") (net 8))
 (segment (start 54.1655 121.62282) (end 54.1655 123.1265) (width 0.254) (layer "F.Cu") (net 8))
 (segment (start 62.996603 123.012199) (end 59.486801 123.012199) (width 0.254) (layer "F.Cu") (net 8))
 (segment (start 62.9285 97.1931) (end 62.9285 96.393) (width 0.508) (layer "F.Cu") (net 8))
 (segment (start 56.769 125.984) (end 56.550561 126.202439) (width 0.254) (layer "F.Cu") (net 8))
 (segment (start 54.1655 123.1265) (end 56.261 125.222) (width 0.254) (layer "F.Cu") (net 8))
 (segment (start 53.745 131.445) (end 52.991 131.445) (width 0.254) (layer "F.Cu") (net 8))
 (segment (start 62.928501 96.393001) (end 62.9285 96.393) (width 0.508) (layer "F.Cu") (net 8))
 (segment (start 58.039 125.222) (end 56.769 125.222) (width 0.254) (layer "F.Cu") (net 8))
 (segment (start 66.944001 119.064801) (end 62.996603 123.012199) (width 0.254) (layer "F.Cu") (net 8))
 (segment (start 57.277 125.222) (end 56.769 125.222) (width 0.254) (layer "F.Cu") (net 8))
 (segment (start 70.9295 95.123) (end 70.929499 96.393001) (width 0.508) (layer "F.Cu") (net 8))
 (segment (start 65.913 118.679) (end 66.817 118.679) (width 0.254) (layer "F.Cu") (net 8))
 (segment (start 59.486801 123.012199) (end 57.277 125.222) (width 0.254) (layer "F.Cu") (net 8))
 (segment (start 56.261 125.222) (end 56.769 125.222) (width 0.254) (layer "F.Cu") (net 8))
 (segment (start 64.713401 113.893599) (end 66.944001 116.124199) (width 0.254) (layer "F.Cu") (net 8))
 (segment (start 53.422551 126.202439) (end 52.6415 126.98349) (width 0.254) (layer "F.Cu") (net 8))
 (segment (start 63.474599 113.893599) (end 64.713401 113.893599) (width 0.254) (layer "F.Cu") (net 8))
 (segment (start 62.484 97.6376) (end 62.9285 97.1931) (width 0.508) (layer "F.Cu") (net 8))
 (segment (start 64.5287 106.553) (end 64.5287 105.283) (width 0.508) (layer "F.Cu") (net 8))
 (segment (start 61.214 97.6376) (end 62.484 97.6376) (width 0.508) (layer "F.Cu") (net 8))
 (segment (start 56.550561 126.202439) (end 53.422551 126.202439) (width 0.254) (layer "F.Cu") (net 8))
 (segment (start 52.991 131.445) (end 52.6415 131.0955) (width 0.254) (layer "F.Cu") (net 8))
 (segment (start 64.5287 105.283) (end 65.7733 104.0384) (width 0.508) (layer "F.Cu") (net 8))
 (segment (start 56.769 125.222) (end 56.769 125.984) (width 0.254) (layer "F.Cu") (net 8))
 (segment (start 66.817 118.679) (end 66.944001 118.806001) (width 0.254) (layer "F.Cu") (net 8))
 (segment (start 70.929499 96.393001) (end 62.928501 96.393001) (width 0.508) (layer "F.Cu") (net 8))
 (segment (start 64.5287 106.553) (end 64.5287 112.333614) (width 0.508) (layer "F.Cu") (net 8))
 (segment (start 59.562989 105.409989) (end 60.071 105.918) (width 0.254) (layer "F.Cu") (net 9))
 (segment (start 60.071 105.918) (end 60.071 110.49) (width 0.254) (layer "F.Cu") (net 9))
 (segment (start 60.198 103.2383) (end 59.562989 103.873311) (width 0.254) (layer "F.Cu") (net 9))
 (segment (start 59.562989 103.873311) (end 59.562989 105.409989) (width 0.254) (layer "F.Cu") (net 9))
 (segment (start 61.214 103.2383) (end 60.198 103.2383) (width 0.254) (layer "F.Cu") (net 9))
 (segment (start 60.071 113.03) (end 61.315601 111.785399) (width 0.254) (layer "F.Cu") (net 10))
 (segment (start 61.315601 111.785399) (end 61.315601 106.444167) (width 0.254) (layer "F.Cu") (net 10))
 (segment (start 60.198 104.0384) (end 61.214 104.0384) (width 0.254) (layer "F.Cu") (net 10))
 (segment (start 61.315601 106.444167) (end 60.070999 105.199565) (width 0.254) (layer "F.Cu") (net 10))
 (segment (start 60.070999 104.165401) (end 60.198 104.0384) (width 0.254) (layer "F.Cu") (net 10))
 (segment (start 60.070999 105.199565) (end 60.070999 104.165401) (width 0.254) (layer "F.Cu") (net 10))
 (segment (start 63.855601 107.696001) (end 63.7286 107.569) (width 0.254) (layer "F.Cu") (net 11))
 (segment (start 62.89 115.479) (end 61.366399 113.955399) (width 0.254) (layer "F.Cu") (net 11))
 (segment (start 60.668409 114.274601) (end 61.366399 113.576611) (width 0.254) (layer "F.Cu") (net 11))
 (segment (start 62.084833 111.734601) (end 63.779401 111.734601) (width 0.254) (layer "F.Cu") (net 11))
 (segment (start 58.826399 112.483389) (end 58.826399 113.627409) (width 0.254) (layer "F.Cu") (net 11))
 (segment (start 58.826399 113.627409) (end 59.473591 114.274601) (width 0.254) (layer "F.Cu") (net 11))
 (segment (start 63.779401 111.734601) (end 63.855601 111.658401) (width 0.254) (layer "F.Cu") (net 11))
 (segment (start 61.366399 113.576611) (end 61.366399 112.453035) (width 0.254) (layer "F.Cu") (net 11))
 (segment (start 59.473591 114.274601) (end 60.668409 114.274601) (width 0.254) (layer "F.Cu") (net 11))
 (segment (start 63.855601 111.658401) (end 63.855601 107.696001) (width 0.254) (layer "F.Cu") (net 11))
 (segment (start 57.531 110.49) (end 57.531 111.18799) (width 0.254) (layer "F.Cu") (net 11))
 (segment (start 63.7286 107.569) (end 63.7286 106.553) (width 0.254) (layer "F.Cu") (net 11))
 (segment (start 63.919 115.479) (end 62.89 115.479) (width 0.254) (layer "F.Cu") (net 11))
 (segment (start 65.913 116.779) (end 65.219 116.779) (width 0.254) (layer "F.Cu") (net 11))
 (segment (start 57.531 111.18799) (end 58.826399 112.483389) (width 0.254) (layer "F.Cu") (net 11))
 (segment (start 61.366399 113.955399) (end 61.366399 113.576611) (width 0.254) (layer "F.Cu") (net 11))
 (segment (start 63.919 119.979) (end 63.919 115.479) (width 0.254) (layer "F.Cu") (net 11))
 (segment (start 65.219 116.779) (end 63.919 115.479) (width 0.254) (layer "F.Cu") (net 11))
 (segment (start 61.366399 112.453035) (end 62.084833 111.734601) (width 0.254) (layer "F.Cu") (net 11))
 (segment (start 53.01488 122.3772) (end 52.91455 122.3772) (width 0.254) (layer "F.Cu") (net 47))
 (segment (start 52.91455 122.3772) (end 52.2605 121.72315) (width 0.254) (layer "F.Cu") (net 47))
 (segment (start 53.594 124.88418) (end 50.82282 124.88418) (width 0.254) (layer "F.Cu") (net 47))
 (segment (start 50.82282 124.88418) (end 50.8 124.907) (width 0.254) (layer "F.Cu") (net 47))
 (segment (start 52.2605 121.72315) (end 52.2605 121.62282) (width 0.254) (layer "F.Cu") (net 47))
 (segment (start 53.594 124.88418) (end 53.594 122.95632) (width 0.254) (layer "F.Cu") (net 47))
 (segment (start 53.594 122.95632) (end 53.01488 122.3772) (width 0.254) (layer "F.Cu") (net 47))
 (segment (start 54.5465 127.08382) (end 56.34482 127.08382) (width 0.254) (layer "F.Cu") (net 46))
 (segment (start 59.438 129.429) (end 57.517 127.508) (width 0.254) (layer "F.Cu") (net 46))
 (segment (start 59.563 129.429) (end 59.438 129.429) (width 0.254) (layer "F.Cu") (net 46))
 (segment (start 57.517 127.508) (end 56.769 127.508) (width 0.254) (layer "F.Cu") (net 46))
 (segment (start 56.34482 127.08382) (end 56.769 127.508) (width 0.254) (layer "F.Cu") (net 46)))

